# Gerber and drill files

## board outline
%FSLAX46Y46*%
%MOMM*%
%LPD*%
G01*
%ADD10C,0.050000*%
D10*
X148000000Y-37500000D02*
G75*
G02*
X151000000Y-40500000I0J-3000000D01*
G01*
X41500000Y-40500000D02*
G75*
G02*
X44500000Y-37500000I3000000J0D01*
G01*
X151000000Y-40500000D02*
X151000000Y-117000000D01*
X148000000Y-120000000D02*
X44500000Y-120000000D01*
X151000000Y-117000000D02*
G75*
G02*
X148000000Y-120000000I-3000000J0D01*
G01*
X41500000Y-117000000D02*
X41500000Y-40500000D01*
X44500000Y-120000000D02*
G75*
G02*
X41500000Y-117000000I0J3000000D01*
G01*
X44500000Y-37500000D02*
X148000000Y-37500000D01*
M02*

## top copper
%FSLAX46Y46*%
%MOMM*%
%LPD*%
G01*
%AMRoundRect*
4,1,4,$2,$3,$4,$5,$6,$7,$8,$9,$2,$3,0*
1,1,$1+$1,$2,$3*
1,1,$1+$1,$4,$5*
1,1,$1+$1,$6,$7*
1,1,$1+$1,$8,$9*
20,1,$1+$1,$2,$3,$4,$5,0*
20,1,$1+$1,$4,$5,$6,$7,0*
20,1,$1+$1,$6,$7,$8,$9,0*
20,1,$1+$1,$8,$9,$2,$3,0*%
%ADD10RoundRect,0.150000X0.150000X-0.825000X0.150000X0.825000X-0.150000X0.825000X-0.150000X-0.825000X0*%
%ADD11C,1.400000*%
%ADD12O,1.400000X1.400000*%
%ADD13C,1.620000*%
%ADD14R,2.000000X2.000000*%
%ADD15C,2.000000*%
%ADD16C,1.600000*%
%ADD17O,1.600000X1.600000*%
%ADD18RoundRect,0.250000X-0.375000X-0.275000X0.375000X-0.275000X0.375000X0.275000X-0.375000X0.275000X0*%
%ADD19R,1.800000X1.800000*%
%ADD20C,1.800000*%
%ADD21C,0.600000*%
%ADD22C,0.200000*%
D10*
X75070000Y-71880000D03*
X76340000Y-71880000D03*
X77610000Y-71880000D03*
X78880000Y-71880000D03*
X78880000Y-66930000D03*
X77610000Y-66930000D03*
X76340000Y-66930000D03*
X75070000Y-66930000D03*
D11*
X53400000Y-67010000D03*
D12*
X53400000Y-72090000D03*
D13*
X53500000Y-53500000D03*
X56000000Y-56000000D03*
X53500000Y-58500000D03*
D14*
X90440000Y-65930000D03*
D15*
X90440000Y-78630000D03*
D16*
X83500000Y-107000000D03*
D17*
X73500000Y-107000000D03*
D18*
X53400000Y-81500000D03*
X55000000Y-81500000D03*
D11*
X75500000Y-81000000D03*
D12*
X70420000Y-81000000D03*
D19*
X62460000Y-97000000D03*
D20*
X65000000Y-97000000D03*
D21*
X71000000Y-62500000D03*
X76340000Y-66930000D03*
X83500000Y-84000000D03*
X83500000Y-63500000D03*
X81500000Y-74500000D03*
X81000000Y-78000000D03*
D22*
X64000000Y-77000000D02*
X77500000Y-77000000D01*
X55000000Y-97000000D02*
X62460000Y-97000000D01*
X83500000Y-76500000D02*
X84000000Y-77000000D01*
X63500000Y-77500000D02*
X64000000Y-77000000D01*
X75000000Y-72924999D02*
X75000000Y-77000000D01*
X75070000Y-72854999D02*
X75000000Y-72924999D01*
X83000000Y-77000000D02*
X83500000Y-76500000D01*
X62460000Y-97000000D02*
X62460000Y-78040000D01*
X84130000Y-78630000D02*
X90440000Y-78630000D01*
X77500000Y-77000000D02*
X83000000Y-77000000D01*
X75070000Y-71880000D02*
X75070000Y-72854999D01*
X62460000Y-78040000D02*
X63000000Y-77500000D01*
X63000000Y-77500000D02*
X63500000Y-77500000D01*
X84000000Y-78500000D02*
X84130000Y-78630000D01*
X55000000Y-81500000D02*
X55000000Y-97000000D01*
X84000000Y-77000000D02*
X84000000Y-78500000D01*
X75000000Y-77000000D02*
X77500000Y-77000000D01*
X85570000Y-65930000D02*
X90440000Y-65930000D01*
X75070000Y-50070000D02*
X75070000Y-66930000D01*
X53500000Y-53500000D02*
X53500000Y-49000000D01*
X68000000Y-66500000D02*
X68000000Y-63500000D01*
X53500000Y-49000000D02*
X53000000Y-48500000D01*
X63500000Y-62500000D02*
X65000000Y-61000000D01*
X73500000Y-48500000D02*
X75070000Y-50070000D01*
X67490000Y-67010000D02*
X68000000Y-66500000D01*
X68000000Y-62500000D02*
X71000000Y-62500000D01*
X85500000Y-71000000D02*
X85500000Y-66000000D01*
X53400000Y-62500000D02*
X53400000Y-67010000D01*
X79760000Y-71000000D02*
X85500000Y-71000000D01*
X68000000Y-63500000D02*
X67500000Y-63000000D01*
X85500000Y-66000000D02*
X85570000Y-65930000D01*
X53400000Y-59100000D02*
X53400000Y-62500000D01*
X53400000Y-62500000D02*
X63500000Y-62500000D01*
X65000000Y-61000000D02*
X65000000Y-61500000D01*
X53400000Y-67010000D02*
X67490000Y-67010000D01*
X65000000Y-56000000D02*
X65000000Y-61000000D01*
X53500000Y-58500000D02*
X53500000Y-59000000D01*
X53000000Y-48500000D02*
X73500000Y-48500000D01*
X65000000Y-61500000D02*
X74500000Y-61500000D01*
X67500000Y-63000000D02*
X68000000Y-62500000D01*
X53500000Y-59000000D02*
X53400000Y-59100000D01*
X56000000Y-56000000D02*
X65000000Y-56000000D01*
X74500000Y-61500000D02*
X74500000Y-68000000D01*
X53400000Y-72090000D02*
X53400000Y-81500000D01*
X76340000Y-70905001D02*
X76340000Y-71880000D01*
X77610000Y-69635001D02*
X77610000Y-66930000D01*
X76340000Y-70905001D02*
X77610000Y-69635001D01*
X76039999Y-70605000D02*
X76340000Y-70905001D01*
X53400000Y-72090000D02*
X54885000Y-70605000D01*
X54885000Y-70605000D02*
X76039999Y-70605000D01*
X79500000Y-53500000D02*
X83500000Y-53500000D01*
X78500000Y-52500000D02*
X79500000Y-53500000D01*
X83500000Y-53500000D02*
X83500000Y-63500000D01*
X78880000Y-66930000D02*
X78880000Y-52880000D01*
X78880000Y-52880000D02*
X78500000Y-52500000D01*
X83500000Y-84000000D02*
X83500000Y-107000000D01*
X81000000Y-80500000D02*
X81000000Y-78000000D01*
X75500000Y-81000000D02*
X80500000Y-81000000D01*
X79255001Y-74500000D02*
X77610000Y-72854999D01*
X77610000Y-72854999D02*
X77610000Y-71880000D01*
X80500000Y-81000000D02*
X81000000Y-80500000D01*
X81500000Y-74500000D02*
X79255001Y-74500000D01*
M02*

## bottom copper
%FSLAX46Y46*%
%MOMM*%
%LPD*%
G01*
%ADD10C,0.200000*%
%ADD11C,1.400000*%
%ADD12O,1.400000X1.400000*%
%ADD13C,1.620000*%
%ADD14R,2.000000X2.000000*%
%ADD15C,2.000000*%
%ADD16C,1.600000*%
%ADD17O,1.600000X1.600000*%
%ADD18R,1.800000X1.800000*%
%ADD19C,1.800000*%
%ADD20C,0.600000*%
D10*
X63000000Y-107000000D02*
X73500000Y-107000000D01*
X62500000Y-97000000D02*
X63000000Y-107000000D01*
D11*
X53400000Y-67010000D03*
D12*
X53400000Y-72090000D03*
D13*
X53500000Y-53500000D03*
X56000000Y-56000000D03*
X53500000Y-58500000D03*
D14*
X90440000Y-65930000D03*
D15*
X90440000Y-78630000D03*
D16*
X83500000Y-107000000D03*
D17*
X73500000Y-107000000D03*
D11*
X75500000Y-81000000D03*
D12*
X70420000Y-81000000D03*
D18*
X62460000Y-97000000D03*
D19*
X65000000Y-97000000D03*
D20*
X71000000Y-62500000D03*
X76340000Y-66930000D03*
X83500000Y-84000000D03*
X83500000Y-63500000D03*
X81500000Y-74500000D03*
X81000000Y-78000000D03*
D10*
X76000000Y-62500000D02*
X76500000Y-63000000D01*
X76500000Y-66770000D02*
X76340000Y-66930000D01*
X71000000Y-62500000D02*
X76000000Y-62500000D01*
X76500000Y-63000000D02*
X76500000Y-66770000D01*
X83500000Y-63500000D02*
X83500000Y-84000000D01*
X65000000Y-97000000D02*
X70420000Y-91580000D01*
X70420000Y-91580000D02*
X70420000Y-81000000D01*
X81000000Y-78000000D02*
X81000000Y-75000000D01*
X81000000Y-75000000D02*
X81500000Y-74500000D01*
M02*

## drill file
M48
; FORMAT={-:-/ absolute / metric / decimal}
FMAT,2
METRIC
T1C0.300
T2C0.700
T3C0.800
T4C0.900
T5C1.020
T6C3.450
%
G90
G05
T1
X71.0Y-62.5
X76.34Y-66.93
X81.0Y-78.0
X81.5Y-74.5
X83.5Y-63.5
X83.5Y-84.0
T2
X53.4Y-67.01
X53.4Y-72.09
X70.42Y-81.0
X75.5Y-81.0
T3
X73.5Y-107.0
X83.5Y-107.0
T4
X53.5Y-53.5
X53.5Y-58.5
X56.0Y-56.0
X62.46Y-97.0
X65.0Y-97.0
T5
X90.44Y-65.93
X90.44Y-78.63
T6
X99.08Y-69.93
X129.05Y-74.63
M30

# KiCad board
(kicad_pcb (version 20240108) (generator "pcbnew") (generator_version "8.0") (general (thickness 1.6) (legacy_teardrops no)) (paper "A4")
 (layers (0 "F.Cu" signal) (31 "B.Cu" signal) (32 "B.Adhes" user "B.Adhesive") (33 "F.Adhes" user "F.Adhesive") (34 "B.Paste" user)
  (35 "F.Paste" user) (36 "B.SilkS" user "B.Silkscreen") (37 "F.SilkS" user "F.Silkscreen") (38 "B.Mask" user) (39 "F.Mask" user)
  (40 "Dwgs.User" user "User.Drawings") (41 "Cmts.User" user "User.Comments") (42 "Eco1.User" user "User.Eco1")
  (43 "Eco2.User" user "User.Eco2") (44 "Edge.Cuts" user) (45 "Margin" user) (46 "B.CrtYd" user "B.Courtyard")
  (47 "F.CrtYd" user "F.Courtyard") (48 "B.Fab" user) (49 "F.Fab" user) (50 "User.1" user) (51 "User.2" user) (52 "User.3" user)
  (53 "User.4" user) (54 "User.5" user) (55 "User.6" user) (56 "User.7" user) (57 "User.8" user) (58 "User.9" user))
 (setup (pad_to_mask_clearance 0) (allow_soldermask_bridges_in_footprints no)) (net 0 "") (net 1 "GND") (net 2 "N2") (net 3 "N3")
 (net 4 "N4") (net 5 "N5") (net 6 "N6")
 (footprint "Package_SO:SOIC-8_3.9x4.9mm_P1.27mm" (layer "F.Cu") (at 76.975 69.405 90)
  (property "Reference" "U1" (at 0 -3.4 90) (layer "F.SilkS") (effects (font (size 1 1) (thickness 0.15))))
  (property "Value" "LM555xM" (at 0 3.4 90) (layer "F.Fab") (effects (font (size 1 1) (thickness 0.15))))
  (pad "1" smd roundrect (at -2.475 -1.905 90) (size 1.95 0.6) (layers "F.Cu" "F.Paste" "F.Mask") (roundrect_rratio 0.25) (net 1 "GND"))
  (pad "2" smd roundrect (at -2.475 -0.635 90) (size 1.95 0.6) (layers "F.Cu" "F.Paste" "F.Mask") (roundrect_rratio 0.25) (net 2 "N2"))
  (pad "3" smd roundrect (at -2.475 0.635 90) (size 1.95 0.6) (layers "F.Cu" "F.Paste" "F.Mask") (roundrect_rratio 0.25) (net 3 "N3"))
  (pad "4" smd roundrect (at -2.475 1.905 90) (size 1.95 0.6) (layers "F.Cu" "F.Paste" "F.Mask") (roundrect_rratio 0.25) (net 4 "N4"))
  (pad "5" smd roundrect (at 2.475 1.905 90) (size 1.95 0.6) (layers "F.Cu" "F.Paste" "F.Mask") (roundrect_rratio 0.25) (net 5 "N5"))
  (pad "6" smd roundrect (at 2.475 0.635 90) (size 1.95 0.6) (layers "F.Cu" "F.Paste" "F.Mask") (roundrect_rratio 0.25) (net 2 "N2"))
  (pad "7" smd roundrect (at 2.475 -0.635 90) (size 1.95 0.6) (layers "F.Cu" "F.Paste" "F.Mask") (roundrect_rratio 0.25) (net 4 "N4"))
  (pad "8" smd roundrect (at 2.475 -1.905 90) (size 1.95 0.6) (layers "F.Cu" "F.Paste" "F.Mask") (roundrect_rratio 0.25) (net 4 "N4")))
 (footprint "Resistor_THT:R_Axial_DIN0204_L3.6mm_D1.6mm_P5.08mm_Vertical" (layer "F.Cu") (at 53.4 67.01 -90)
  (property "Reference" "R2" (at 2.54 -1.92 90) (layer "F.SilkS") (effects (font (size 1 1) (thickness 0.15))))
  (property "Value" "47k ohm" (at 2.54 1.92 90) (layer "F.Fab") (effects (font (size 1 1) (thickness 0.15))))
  (pad "1" thru_hole circle (at 0 0 270) (size 1.4 1.4) (drill 0.7) (layers "*.Cu" "*.Mask") (remove_unused_layers no) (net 4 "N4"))
  (pad "2" thru_hole oval (at 5.08 0 270) (size 1.4 1.4) (drill 0.7) (layers "*.Cu" "*.Mask") (remove_unused_layers no) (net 2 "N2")))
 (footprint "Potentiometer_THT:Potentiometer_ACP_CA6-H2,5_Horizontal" (layer "F.Cu") (at 53.5 53.5)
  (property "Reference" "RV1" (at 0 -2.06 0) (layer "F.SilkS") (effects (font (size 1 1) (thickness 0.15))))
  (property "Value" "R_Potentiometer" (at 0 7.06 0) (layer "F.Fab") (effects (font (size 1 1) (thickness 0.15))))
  (pad "1" thru_hole circle (at 0 0) (size 1.62 1.62) (drill 0.9) (layers "*.Cu" "*.Mask") (remove_unused_layers no) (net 4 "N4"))
  (pad "2" thru_hole circle (at 2.5 2.5) (size 1.62 1.62) (drill 0.9) (layers "*.Cu" "*.Mask") (remove_unused_layers no) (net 4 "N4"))
  (pad "3" thru_hole circle (at 0 5) (size 1.62 1.62) (drill 0.9) (layers "*.Cu" "*.Mask") (remove_unused_layers no) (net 4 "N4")))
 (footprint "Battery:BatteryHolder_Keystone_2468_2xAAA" (layer "F.Cu") (at 90.44 65.93)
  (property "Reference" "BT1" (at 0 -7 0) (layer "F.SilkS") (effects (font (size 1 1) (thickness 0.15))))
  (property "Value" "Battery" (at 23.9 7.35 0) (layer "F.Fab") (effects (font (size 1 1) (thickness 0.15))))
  (pad "" np_thru_hole circle (at 8.64 4) (size 3.45 3.45) (drill 3.45) (layers "*.Cu"))
  (pad "" np_thru_hole circle (at 38.61 8.7) (size 3.45 3.45) (drill 3.45) (layers "*.Cu" "*.Mask"))
  (pad "1" thru_hole rect (at 0 0) (size 2 2) (drill 1.02) (layers "*.Cu" "*.Mask") (remove_unused_layers no) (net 4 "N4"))
  (pad "2" thru_hole circle (at 0 12.7) (size 2 2) (drill 1.02) (layers "*.Cu" "*.Mask") (remove_unused_layers no) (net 1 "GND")))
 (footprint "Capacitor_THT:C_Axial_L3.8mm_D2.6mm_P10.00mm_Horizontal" (layer "F.Cu") (at 83.5 107 180)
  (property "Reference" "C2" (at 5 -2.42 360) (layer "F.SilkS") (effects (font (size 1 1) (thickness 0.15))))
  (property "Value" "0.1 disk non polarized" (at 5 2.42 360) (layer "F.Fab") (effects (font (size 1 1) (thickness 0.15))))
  (pad "1" thru_hole circle (at 0 0 180) (size 1.6 1.6) (drill 0.8) (layers "*.Cu" "*.Mask") (remove_unused_layers no) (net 5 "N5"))
  (pad "2" thru_hole oval (at 10 0 180) (size 1.6 1.6) (drill 0.8) (layers "*.Cu" "*.Mask") (remove_unused_layers no) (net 1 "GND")))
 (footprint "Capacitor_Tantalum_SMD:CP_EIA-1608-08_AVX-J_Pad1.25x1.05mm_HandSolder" (layer "F.Cu") (at 54.2 81.5)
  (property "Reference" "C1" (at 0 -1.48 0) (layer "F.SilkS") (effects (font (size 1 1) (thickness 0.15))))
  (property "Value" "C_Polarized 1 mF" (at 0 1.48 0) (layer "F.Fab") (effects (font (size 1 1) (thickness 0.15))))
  (pad "1" smd roundrect (at -0.8 0) (size 1.25 1.05) (layers "F.Cu" "F.Paste" "F.Mask") (roundrect_rratio 0.238095) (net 2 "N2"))
  (pad "2" smd roundrect (at 0.8 0) (size 1.25 1.05) (layers "F.Cu" "F.Paste" "F.Mask") (roundrect_rratio 0.238095) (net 1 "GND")))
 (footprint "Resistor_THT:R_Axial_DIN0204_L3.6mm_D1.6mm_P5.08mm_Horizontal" (layer "F.Cu") (at 75.5 81 180)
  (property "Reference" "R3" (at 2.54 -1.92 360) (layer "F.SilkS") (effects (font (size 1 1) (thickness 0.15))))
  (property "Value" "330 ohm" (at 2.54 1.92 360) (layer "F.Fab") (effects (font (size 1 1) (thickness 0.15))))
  (pad "1" thru_hole circle (at 0 0 180) (size 1.4 1.4) (drill 0.7) (layers "*.Cu" "*.Mask") (remove_unused_layers no) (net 3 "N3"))
  (pad "2" thru_hole oval (at 5.08 0 180) (size 1.4 1.4) (drill 0.7) (layers "*.Cu" "*.Mask") (remove_unused_layers no) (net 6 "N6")))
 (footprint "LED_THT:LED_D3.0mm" (layer "F.Cu") (at 62.46 97)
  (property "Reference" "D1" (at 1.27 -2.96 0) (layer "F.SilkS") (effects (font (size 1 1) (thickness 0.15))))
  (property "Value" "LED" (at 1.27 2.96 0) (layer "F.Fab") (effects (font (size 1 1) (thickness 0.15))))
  (pad "1" thru_hole rect (at 0 0) (size 1.8 1.8) (drill 0.9) (layers "*.Cu" "*.Mask") (remove_unused_layers no) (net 1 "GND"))
  (pad "2" thru_hole circle (at 2.54 0) (size 1.8 1.8) (drill 0.9) (layers "*.Cu" "*.Mask") (remove_unused_layers no) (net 6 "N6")))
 (gr_line (start 63 107) (end 73.5 107) (stroke (width 0.2) (type default)) (layer "B.Cu") (net 1))
 (gr_line (start 62.5 97) (end 63 107) (stroke (width 0.2) (type default)) (layer "B.Cu") (net 1))
 (gr_arc (start 148 37.5) (mid 150.12132 38.37868) (end 151 40.5) (stroke (width 0.05) (type default)) (layer "Edge.Cuts"))
 (gr_arc (start 41.5 40.5) (mid 42.37868 38.37868) (end 44.5 37.5) (stroke (width 0.05) (type default)) (layer "Edge.Cuts"))
 (gr_line (start 151 40.5) (end 151 117) (stroke (width 0.05) (type default)) (layer "Edge.Cuts"))
 (gr_line (start 148 120) (end 44.5 120) (stroke (width 0.05) (type default)) (layer "Edge.Cuts"))
 (gr_arc (start 151 117) (mid 150.12132 119.12132) (end 148 120) (stroke (width 0.05) (type default)) (layer "Edge.Cuts"))
 (gr_line (start 41.5 117) (end 41.5 40.5) (stroke (width 0.05) (type default)) (layer "Edge.Cuts"))
 (gr_arc (start 44.5 120) (mid 42.37868 119.12132) (end 41.5 117) (stroke (width 0.05) (type default)) (layer "Edge.Cuts"))
 (gr_line (start 44.5 37.5) (end 148 37.5) (stroke (width 0.05) (type default)) (layer "Edge.Cuts"))
 (segment (start 64 77) (end 77.5 77) (width 0.2) (layer "F.Cu") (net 1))
 (segment (start 55 97) (end 62.46 97) (width 0.2) (layer "F.Cu") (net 1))
 (segment (start 83.5 76.5) (end 84 77) (width 0.2) (layer "F.Cu") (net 1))
 (segment (start 63.5 77.5) (end 64 77) (width 0.2) (layer "F.Cu") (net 1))
 (segment (start 75 72.924999) (end 75 77) (width 0.2) (layer "F.Cu") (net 1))
 (segment (start 75.07 72.854999) (end 75 72.924999) (width 0.2) (layer "F.Cu") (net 1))
 (segment (start 83 77) (end 83.5 76.5) (width 0.2) (layer "F.Cu") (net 1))
 (segment (start 62.46 97) (end 62.46 78.04) (width 0.2) (layer "F.Cu") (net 1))
 (segment (start 84.13 78.63) (end 90.44 78.63) (width 0.2) (layer "F.Cu") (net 1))
 (segment (start 77.5 77) (end 83 77) (width 0.2) (layer "F.Cu") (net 1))
 (segment (start 75.07 71.88) (end 75.07 72.854999) (width 0.2) (layer "F.Cu") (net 1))
 (segment (start 62.46 78.04) (end 63 77.5) (width 0.2) (layer "F.Cu") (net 1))
 (segment (start 63 77.5) (end 63.5 77.5) (width 0.2) (layer "F.Cu") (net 1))
 (segment (start 84 78.5) (end 84.13 78.63) (width 0.2) (layer "F.Cu") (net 1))
 (segment (start 55 81.5) (end 55 97) (width 0.2) (layer "F.Cu") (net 1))
 (segment (start 84 77) (end 84 78.5) (width 0.2) (layer "F.Cu") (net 1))
 (segment (start 75 77) (end 77.5 77) (width 0.2) (layer "F.Cu") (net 1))
 (segment (start 85.57 65.93) (end 90.44 65.93) (width 0.2) (layer "F.Cu") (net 4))
 (segment (start 75.07 50.07) (end 75.07 66.93) (width 0.2) (layer "F.Cu") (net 4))
 (segment (start 53.5 53.5) (end 53.5 49) (width 0.2) (layer "F.Cu") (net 4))
 (segment (start 68 66.5) (end 68 63.5) (width 0.2) (layer "F.Cu") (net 4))
 (segment (start 53.5 49) (end 53 48.5) (width 0.2) (layer "F.Cu") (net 4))
 (segment (start 63.5 62.5) (end 65 61) (width 0.2) (layer "F.Cu") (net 4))
 (segment (start 73.5 48.5) (end 75.07 50.07) (width 0.2) (layer "F.Cu") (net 4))
 (segment (start 67.49 67.01) (end 68 66.5) (width 0.2) (layer "F.Cu") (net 4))
 (segment (start 68 62.5) (end 71 62.5) (width 0.2) (layer "F.Cu") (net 4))
 (segment (start 85.5 71) (end 85.5 66) (width 0.2) (layer "F.Cu") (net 4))
 (segment (start 53.4 62.5) (end 53.4 67.01) (width 0.2) (layer "F.Cu") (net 4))
 (segment (start 79.76 71) (end 85.5 71) (width 0.2) (layer "F.Cu") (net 4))
 (segment (start 68 63.5) (end 67.5 63) (width 0.2) (layer "F.Cu") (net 4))
 (segment (start 85.5 66) (end 85.57 65.93) (width 0.2) (layer "F.Cu") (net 4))
 (segment (start 53.4 59.1) (end 53.4 62.5) (width 0.2) (layer "F.Cu") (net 4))
 (segment (start 53.4 62.5) (end 63.5 62.5) (width 0.2) (layer "F.Cu") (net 4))
 (segment (start 65 61) (end 65 61.5) (width 0.2) (layer "F.Cu") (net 4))
 (segment (start 53.4 67.01) (end 67.49 67.01) (width 0.2) (layer "F.Cu") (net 4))
 (segment (start 65 56) (end 65 61) (width 0.2) (layer "F.Cu") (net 4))
 (segment (start 53.5 58.5) (end 53.5 59) (width 0.2) (layer "F.Cu") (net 4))
 (segment (start 53 48.5) (end 73.5 48.5) (width 0.2) (layer "F.Cu") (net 4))
 (segment (start 65 61.5) (end 74.5 61.5) (width 0.2) (layer "F.Cu") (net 4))
 (segment (start 67.5 63) (end 68 62.5) (width 0.2) (layer "F.Cu") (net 4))
 (segment (start 53.5 59) (end 53.4 59.1) (width 0.2) (layer "F.Cu") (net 4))
 (segment (start 56 56) (end 65 56) (width 0.2) (layer "F.Cu") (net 4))
 (segment (start 74.5 61.5) (end 74.5 68) (width 0.2) (layer "F.Cu") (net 4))
 (via (at 71 62.5) (size 0.6) (drill 0.3) (layers "F.Cu" "B.Cu") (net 4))
 (via (at 76.34 66.93) (size 0.6) (drill 0.3) (layers "F.Cu" "B.Cu") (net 4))
 (segment (start 76 62.5) (end 76.5 63) (width 0.2) (layer "B.Cu") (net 4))
 (segment (start 76.5 66.77) (end 76.34 66.93) (width 0.2) (layer "B.Cu") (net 4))
 (segment (start 71 62.5) (end 76 62.5) (width 0.2) (layer "B.Cu") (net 4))
 (segment (start 76.5 63) (end 76.5 66.77) (width 0.2) (layer "B.Cu") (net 4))
 (segment (start 53.4 72.09) (end 53.4 81.5) (width 0.2) (layer "F.Cu") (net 2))
 (segment (start 76.34 70.905001) (end 76.34 71.88) (width 0.2) (layer "F.Cu") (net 2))
 (segment (start 77.61 69.635001) (end 77.61 66.93) (width 0.2) (layer "F.Cu") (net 2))
 (segment (start 76.34 70.905001) (end 77.61 69.635001) (width 0.2) (layer "F.Cu") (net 2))
 (segment (start 76.039999 70.605) (end 76.34 70.905001) (width 0.2) (layer "F.Cu") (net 2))
 (segment (start 53.4 72.09) (end 54.885 70.605) (width 0.2) (layer "F.Cu") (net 2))
 (segment (start 54.885 70.605) (end 76.039999 70.605) (width 0.2) (layer "F.Cu") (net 2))
 (segment (start 79.5 53.5) (end 83.5 53.5) (width 0.2) (layer "F.Cu") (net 5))
 (segment (start 78.5 52.5) (end 79.5 53.5) (width 0.2) (layer "F.Cu") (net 5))
 (segment (start 83.5 53.5) (end 83.5 63.5) (width 0.2) (layer "F.Cu") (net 5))
 (segment (start 78.88 66.93) (end 78.88 52.88) (width 0.2) (layer "F.Cu") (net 5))
 (segment (start 78.88 52.88) (end 78.5 52.5) (width 0.2) (layer "F.Cu") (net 5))
 (segment (start 83.5 84) (end 83.5 107) (width 0.2) (layer "F.Cu") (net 5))
 (via (at 83.5 84) (size 0.6) (drill 0.3) (layers "F.Cu" "B.Cu") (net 5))
 (via (at 83.5 63.5) (size 0.6) (drill 0.3) (layers "F.Cu" "B.Cu") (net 5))
 (segment (start 83.5 63.5) (end 83.5 84) (width 0.2) (layer "B.Cu") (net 5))
 (segment (start 65 97) (end 70.42 91.58) (width 0.2) (layer "B.Cu") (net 6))
 (segment (start 70.42 91.58) (end 70.42 81) (width 0.2) (layer "B.Cu") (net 6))
 (segment (start 81 80.5) (end 81 78) (width 0.2) (layer "F.Cu") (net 3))
 (segment (start 75.5 81) (end 80.5 81) (width 0.2) (layer "F.Cu") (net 3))
 (segment (start 79.255001 74.5) (end 77.61 72.854999) (width 0.2) (layer "F.Cu") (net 3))
 (segment (start 77.61 72.854999) (end 77.61 71.88) (width 0.2) (layer "F.Cu") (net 3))
 (segment (start 80.5 81) (end 81 80.5) (width 0.2) (layer "F.Cu") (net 3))
 (segment (start 81.5 74.5) (end 79.255001 74.5) (width 0.2) (layer "F.Cu") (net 3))
 (via (at 81.5 74.5) (size 0.6) (drill 0.3) (layers "F.Cu" "B.Cu") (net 3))
 (via (at 81 78) (size 0.6) (drill 0.3) (layers "F.Cu" "B.Cu") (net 3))
 (segment (start 81 78) (end 81 75) (width 0.2) (layer "B.Cu") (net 3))
 (segment (start 81 75) (end 81.5 74.5) (width 0.2) (layer "B.Cu") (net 3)))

